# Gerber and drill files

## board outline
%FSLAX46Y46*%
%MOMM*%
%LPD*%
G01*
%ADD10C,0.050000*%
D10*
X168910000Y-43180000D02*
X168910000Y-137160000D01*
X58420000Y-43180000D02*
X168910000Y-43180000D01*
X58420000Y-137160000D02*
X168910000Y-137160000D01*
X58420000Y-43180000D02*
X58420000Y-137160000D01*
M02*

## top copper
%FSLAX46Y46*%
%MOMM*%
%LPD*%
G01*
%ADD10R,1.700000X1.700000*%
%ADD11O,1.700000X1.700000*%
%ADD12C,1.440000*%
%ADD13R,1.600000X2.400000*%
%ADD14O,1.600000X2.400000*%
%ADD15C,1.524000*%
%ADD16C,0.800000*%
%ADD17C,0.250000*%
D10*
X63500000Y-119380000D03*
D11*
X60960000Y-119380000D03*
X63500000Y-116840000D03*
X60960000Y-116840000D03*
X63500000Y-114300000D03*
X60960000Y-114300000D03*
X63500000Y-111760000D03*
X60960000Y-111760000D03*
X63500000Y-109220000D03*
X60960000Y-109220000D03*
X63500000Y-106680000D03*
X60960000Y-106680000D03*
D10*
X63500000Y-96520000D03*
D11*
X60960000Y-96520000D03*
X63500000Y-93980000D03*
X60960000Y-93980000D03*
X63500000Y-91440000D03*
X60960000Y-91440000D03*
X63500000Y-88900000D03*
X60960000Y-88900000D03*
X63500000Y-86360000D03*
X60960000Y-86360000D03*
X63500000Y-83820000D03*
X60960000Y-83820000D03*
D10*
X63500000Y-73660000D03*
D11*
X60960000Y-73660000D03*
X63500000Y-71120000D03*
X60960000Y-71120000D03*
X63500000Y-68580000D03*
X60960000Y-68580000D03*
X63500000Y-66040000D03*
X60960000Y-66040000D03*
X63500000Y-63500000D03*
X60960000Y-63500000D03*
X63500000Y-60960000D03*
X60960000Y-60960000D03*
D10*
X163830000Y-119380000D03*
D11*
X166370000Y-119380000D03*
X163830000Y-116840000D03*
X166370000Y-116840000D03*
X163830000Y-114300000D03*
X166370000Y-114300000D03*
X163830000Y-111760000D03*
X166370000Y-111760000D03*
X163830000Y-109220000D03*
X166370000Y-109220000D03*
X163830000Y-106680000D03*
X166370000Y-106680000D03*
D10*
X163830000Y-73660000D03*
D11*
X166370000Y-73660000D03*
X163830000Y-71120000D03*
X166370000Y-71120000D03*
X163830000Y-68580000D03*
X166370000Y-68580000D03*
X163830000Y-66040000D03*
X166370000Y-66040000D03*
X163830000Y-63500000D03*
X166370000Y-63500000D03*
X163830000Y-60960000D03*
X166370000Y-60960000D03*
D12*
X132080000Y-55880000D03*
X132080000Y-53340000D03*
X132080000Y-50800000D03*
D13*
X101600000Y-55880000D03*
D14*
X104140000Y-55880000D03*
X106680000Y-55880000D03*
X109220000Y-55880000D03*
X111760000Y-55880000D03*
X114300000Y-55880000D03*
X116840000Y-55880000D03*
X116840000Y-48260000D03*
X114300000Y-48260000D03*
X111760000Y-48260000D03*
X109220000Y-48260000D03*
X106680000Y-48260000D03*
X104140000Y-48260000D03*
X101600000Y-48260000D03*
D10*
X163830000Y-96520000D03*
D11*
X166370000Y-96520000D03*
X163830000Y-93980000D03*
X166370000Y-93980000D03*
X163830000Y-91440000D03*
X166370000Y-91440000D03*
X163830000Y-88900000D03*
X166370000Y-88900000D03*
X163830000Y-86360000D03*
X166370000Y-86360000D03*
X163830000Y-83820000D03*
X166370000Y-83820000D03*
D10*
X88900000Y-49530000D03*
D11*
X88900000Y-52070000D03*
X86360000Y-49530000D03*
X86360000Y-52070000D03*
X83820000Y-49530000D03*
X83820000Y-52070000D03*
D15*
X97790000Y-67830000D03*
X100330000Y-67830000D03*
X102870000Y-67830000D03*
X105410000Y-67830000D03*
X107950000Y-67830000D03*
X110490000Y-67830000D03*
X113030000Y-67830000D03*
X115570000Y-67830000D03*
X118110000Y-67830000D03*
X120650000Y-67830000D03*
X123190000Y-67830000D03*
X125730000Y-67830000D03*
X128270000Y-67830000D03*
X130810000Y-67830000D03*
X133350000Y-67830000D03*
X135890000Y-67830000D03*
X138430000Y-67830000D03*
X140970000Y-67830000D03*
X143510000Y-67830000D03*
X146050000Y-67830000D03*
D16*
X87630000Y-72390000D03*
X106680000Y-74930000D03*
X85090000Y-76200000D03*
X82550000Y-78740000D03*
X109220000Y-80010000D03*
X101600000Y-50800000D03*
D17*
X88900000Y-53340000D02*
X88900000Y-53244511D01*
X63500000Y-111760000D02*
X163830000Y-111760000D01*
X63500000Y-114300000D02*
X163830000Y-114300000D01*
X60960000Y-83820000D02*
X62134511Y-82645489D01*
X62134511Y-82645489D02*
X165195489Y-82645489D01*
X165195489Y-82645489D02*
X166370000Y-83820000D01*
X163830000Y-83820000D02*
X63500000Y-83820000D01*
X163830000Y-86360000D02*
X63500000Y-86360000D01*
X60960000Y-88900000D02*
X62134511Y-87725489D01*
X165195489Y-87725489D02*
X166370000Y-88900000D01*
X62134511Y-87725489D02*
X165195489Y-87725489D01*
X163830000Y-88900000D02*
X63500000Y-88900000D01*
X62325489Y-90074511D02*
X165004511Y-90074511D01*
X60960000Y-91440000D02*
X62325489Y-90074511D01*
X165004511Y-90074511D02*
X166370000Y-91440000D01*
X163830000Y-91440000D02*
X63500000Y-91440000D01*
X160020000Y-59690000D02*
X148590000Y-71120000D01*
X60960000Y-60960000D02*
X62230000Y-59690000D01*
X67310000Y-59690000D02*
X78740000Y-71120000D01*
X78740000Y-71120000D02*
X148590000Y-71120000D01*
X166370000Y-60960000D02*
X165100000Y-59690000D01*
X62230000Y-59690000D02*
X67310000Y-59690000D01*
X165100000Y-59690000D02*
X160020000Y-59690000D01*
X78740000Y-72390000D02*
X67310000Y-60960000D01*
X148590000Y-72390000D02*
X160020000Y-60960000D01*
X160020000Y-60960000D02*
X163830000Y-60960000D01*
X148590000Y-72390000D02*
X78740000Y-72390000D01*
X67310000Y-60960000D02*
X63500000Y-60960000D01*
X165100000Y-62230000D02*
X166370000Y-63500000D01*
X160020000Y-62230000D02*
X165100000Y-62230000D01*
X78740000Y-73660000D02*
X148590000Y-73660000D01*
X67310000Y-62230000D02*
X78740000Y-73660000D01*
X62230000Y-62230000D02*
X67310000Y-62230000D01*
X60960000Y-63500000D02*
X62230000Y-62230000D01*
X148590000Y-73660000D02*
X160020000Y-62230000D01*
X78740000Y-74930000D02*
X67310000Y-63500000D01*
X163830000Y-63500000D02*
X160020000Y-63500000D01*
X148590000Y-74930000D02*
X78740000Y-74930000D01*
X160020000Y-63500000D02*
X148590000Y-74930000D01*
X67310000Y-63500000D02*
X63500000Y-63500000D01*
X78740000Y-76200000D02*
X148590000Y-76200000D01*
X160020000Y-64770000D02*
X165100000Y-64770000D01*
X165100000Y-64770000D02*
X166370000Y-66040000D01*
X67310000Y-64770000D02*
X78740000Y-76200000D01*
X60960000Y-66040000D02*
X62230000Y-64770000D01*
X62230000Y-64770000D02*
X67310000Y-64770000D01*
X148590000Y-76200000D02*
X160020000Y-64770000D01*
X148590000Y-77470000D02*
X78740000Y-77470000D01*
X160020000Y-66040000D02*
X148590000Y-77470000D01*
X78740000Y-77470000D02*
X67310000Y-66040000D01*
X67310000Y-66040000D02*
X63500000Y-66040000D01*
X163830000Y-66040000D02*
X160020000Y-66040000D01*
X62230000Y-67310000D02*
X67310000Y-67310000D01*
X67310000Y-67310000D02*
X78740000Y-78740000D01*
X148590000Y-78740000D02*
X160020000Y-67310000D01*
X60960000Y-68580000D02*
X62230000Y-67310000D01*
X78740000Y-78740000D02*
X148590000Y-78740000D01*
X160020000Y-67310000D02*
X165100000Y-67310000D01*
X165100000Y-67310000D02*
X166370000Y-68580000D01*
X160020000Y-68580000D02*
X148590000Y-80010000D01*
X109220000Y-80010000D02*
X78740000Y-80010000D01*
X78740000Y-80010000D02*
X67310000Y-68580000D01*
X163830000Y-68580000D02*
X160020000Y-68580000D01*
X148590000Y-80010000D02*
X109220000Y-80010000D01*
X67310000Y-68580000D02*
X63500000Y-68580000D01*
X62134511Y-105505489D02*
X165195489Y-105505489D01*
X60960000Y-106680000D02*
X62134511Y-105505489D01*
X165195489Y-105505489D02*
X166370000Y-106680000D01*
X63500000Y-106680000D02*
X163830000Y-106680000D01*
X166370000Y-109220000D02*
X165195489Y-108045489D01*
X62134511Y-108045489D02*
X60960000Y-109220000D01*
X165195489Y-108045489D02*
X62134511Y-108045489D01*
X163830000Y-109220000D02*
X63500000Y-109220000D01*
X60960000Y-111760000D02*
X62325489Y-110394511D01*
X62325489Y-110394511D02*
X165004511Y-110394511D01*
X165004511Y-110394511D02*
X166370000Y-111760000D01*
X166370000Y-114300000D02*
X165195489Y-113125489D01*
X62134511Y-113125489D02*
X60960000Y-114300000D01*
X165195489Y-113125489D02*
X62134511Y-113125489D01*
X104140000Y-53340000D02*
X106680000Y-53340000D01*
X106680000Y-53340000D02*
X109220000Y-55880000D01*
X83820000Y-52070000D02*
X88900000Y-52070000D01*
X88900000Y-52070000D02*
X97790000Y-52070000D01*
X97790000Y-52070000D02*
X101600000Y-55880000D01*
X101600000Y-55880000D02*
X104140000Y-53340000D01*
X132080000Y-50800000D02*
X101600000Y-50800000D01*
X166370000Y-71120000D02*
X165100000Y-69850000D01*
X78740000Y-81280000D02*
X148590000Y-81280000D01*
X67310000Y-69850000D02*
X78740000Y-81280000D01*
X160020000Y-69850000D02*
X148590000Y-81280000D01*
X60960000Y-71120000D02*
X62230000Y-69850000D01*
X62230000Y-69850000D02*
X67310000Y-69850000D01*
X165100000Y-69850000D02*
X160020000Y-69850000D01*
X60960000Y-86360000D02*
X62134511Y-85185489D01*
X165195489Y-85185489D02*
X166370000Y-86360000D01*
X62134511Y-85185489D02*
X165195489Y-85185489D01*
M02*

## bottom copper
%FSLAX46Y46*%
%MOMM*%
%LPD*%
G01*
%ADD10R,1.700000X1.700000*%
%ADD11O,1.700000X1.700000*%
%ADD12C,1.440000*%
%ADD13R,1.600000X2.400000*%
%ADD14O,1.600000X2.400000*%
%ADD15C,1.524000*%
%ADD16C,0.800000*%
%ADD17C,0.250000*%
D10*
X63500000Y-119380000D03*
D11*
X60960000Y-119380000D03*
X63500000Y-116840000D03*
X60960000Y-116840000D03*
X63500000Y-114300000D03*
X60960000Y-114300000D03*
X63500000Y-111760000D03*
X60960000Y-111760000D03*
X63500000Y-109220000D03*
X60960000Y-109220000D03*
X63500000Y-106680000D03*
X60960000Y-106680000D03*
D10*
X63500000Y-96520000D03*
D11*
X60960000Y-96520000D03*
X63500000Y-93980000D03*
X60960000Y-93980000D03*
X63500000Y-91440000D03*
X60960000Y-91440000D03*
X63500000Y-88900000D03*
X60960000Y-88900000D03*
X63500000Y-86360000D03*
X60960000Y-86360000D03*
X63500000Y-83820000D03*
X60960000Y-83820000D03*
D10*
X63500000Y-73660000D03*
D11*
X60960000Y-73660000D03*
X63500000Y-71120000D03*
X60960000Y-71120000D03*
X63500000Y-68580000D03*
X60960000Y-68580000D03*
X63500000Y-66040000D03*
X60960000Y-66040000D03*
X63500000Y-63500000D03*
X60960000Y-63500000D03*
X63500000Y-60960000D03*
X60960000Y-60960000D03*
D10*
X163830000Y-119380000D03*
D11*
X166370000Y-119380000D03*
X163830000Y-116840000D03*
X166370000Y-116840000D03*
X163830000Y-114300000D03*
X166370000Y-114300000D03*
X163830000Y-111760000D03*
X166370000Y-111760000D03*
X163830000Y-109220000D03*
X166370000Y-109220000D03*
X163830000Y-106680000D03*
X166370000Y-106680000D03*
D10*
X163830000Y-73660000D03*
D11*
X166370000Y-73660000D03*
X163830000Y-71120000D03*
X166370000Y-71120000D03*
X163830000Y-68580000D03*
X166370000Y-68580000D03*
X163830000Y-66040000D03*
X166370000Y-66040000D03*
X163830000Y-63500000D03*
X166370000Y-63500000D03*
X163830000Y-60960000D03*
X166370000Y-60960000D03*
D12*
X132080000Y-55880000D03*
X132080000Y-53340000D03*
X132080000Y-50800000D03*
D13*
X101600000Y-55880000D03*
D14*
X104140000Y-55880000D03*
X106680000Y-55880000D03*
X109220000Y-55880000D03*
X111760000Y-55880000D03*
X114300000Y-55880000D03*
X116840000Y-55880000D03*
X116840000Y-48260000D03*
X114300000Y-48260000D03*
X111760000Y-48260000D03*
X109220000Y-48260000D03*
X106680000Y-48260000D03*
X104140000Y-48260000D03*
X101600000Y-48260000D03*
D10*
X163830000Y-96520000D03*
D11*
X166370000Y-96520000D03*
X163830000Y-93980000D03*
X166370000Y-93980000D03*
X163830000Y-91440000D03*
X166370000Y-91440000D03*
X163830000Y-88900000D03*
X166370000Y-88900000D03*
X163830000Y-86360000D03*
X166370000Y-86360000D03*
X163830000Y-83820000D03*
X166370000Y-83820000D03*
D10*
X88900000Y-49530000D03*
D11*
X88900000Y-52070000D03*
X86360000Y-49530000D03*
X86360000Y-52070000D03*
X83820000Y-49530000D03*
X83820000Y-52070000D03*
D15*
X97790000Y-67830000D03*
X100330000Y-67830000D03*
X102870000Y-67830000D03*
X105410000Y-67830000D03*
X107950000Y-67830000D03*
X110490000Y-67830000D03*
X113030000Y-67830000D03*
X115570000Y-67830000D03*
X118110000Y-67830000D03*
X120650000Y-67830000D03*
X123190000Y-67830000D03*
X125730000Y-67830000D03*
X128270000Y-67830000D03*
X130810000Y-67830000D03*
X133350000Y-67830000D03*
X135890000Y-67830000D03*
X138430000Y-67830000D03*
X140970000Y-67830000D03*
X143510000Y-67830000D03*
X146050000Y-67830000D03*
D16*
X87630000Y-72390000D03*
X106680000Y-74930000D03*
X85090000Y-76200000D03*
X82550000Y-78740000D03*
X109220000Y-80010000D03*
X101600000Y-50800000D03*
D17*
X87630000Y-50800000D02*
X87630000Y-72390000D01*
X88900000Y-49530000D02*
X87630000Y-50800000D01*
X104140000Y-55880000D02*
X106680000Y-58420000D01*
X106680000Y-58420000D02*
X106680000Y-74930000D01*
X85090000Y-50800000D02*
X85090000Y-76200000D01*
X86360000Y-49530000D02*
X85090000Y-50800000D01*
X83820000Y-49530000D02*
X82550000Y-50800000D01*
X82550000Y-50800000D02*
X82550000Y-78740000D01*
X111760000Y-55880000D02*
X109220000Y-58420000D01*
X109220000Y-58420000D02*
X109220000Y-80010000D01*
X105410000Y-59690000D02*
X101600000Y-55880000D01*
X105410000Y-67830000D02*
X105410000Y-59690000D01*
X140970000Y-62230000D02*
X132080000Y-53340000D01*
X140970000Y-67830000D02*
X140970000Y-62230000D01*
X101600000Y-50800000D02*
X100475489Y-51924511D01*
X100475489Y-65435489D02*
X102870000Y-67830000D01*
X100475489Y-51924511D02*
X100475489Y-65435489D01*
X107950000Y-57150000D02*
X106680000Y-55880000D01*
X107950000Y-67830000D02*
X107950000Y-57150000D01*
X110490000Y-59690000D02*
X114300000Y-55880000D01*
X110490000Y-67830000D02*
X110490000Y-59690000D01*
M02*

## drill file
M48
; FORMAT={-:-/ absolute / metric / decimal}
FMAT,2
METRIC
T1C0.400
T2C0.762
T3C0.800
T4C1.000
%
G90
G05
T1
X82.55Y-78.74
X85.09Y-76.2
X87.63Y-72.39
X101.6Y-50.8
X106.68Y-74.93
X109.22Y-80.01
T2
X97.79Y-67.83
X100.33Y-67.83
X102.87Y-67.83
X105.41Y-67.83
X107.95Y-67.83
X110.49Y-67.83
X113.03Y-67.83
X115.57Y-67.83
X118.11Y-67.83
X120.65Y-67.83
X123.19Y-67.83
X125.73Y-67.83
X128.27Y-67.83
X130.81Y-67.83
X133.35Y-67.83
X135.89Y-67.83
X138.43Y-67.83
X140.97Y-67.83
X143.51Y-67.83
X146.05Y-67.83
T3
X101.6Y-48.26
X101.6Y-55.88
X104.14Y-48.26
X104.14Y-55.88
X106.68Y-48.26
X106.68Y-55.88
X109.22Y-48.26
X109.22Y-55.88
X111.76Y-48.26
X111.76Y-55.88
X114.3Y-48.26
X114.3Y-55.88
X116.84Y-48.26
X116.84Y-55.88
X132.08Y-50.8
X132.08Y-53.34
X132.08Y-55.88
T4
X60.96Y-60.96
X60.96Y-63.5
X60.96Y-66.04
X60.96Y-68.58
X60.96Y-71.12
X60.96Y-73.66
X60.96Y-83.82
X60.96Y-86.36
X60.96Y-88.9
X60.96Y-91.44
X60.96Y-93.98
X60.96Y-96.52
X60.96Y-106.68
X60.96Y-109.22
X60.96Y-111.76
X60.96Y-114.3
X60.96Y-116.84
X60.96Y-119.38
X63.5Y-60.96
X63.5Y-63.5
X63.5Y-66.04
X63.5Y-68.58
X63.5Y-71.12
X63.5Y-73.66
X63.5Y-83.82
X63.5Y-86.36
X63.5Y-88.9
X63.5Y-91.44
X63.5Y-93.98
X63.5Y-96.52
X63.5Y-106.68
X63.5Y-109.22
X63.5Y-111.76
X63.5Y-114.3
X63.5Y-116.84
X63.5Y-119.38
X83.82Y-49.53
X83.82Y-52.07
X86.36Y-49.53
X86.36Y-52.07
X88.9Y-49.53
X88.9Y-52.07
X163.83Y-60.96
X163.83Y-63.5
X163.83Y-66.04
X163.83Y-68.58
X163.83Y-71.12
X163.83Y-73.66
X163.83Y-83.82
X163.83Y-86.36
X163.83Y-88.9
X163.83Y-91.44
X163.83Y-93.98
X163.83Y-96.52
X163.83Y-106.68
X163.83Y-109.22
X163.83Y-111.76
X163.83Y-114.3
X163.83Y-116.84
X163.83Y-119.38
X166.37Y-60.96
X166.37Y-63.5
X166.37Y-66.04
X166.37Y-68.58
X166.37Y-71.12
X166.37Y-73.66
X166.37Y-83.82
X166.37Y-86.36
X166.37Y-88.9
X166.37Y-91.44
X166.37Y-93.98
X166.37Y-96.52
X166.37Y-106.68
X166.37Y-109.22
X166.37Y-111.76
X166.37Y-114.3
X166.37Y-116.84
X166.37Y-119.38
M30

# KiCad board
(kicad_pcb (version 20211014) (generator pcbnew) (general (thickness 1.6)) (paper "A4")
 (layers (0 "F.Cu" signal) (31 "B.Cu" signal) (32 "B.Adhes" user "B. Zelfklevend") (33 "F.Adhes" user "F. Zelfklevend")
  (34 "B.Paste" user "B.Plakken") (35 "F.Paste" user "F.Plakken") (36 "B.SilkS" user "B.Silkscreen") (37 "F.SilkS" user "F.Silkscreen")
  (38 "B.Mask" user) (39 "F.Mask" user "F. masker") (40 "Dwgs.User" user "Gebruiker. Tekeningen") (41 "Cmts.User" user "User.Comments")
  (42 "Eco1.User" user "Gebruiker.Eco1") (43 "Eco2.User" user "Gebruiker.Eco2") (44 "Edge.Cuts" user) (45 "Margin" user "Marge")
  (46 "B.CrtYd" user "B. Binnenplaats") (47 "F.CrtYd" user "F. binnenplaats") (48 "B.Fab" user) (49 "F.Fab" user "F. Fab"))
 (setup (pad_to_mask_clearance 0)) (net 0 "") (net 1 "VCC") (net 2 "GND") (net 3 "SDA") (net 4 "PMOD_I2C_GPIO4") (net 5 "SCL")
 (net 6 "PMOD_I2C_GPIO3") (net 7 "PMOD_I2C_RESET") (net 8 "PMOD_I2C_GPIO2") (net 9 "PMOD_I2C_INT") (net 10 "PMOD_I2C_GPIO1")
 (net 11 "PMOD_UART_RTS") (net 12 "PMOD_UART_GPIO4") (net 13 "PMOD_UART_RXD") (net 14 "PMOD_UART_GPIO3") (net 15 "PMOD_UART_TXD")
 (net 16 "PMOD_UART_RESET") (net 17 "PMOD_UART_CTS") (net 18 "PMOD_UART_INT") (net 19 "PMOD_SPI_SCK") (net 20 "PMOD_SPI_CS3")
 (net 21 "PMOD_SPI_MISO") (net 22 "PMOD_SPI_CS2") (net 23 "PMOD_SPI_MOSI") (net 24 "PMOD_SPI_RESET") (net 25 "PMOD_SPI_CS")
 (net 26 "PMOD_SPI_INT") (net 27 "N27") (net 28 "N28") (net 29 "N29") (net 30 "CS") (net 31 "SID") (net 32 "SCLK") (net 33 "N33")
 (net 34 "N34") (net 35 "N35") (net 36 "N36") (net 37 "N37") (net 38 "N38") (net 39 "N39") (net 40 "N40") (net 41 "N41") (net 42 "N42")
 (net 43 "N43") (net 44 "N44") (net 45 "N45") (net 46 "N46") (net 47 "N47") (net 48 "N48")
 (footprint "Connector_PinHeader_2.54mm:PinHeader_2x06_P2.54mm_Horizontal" (layer "F.Cu") (at 63.5 119.38 180)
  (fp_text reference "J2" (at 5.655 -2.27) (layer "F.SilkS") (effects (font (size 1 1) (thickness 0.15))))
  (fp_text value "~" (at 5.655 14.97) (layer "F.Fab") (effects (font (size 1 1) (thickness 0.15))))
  (pad "1" thru_hole rect (at 0 0 180) (size 1.7 1.7) (drill 1) (layers *.Cu *.Mask) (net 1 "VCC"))
  (pad "2" thru_hole oval (at 2.54 0 180) (size 1.7 1.7) (drill 1) (layers *.Cu *.Mask) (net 1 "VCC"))
  (pad "3" thru_hole oval (at 0 2.54 180) (size 1.7 1.7) (drill 1) (layers *.Cu *.Mask) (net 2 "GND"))
  (pad "4" thru_hole oval (at 2.54 2.54 180) (size 1.7 1.7) (drill 1) (layers *.Cu *.Mask) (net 2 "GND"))
  (pad "5" thru_hole oval (at 0 5.08 180) (size 1.7 1.7) (drill 1) (layers *.Cu *.Mask) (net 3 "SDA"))
  (pad "6" thru_hole oval (at 2.54 5.08 180) (size 1.7 1.7) (drill 1) (layers *.Cu *.Mask) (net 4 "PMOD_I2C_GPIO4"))
  (pad "7" thru_hole oval (at 0 7.62 180) (size 1.7 1.7) (drill 1) (layers *.Cu *.Mask) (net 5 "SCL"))
  (pad "8" thru_hole oval (at 2.54 7.62 180) (size 1.7 1.7) (drill 1) (layers *.Cu *.Mask) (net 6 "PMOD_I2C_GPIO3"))
  (pad "9" thru_hole oval (at 0 10.16 180) (size 1.7 1.7) (drill 1) (layers *.Cu *.Mask) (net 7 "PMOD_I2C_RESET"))
  (pad "10" thru_hole oval (at 2.54 10.16 180) (size 1.7 1.7) (drill 1) (layers *.Cu *.Mask) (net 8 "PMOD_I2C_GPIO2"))
  (pad "11" thru_hole oval (at 0 12.7 180) (size 1.7 1.7) (drill 1) (layers *.Cu *.Mask) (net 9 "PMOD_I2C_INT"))
  (pad "12" thru_hole oval (at 2.54 12.7 180) (size 1.7 1.7) (drill 1) (layers *.Cu *.Mask) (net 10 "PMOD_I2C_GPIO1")))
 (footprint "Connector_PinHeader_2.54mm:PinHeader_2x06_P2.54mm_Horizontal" (layer "F.Cu") (at 63.5 96.52 180)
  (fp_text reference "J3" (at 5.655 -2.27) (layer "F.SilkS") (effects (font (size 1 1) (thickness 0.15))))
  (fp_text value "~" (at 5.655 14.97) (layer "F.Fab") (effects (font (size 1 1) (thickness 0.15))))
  (pad "1" thru_hole rect (at 0 0 180) (size 1.7 1.7) (drill 1) (layers *.Cu *.Mask) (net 1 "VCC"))
  (pad "2" thru_hole oval (at 2.54 0 180) (size 1.7 1.7) (drill 1) (layers *.Cu *.Mask) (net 1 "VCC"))
  (pad "3" thru_hole oval (at 0 2.54 180) (size 1.7 1.7) (drill 1) (layers *.Cu *.Mask) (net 2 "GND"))
  (pad "4" thru_hole oval (at 2.54 2.54 180) (size 1.7 1.7) (drill 1) (layers *.Cu *.Mask) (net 2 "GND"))
  (pad "5" thru_hole oval (at 0 5.08 180) (size 1.7 1.7) (drill 1) (layers *.Cu *.Mask) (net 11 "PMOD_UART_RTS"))
  (pad "6" thru_hole oval (at 2.54 5.08 180) (size 1.7 1.7) (drill 1) (layers *.Cu *.Mask) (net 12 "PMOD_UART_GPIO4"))
  (pad "7" thru_hole oval (at 0 7.62 180) (size 1.7 1.7) (drill 1) (layers *.Cu *.Mask) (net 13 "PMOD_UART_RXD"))
  (pad "8" thru_hole oval (at 2.54 7.62 180) (size 1.7 1.7) (drill 1) (layers *.Cu *.Mask) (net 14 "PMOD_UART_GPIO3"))
  (pad "9" thru_hole oval (at 0 10.16 180) (size 1.7 1.7) (drill 1) (layers *.Cu *.Mask) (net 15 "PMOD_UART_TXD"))
  (pad "10" thru_hole oval (at 2.54 10.16 180) (size 1.7 1.7) (drill 1) (layers *.Cu *.Mask) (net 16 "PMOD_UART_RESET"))
  (pad "11" thru_hole oval (at 0 12.7 180) (size 1.7 1.7) (drill 1) (layers *.Cu *.Mask) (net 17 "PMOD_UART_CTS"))
  (pad "12" thru_hole oval (at 2.54 12.7 180) (size 1.7 1.7) (drill 1) (layers *.Cu *.Mask) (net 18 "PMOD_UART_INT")))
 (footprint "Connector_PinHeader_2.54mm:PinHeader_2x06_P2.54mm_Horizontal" (layer "F.Cu") (at 63.5 73.66 180)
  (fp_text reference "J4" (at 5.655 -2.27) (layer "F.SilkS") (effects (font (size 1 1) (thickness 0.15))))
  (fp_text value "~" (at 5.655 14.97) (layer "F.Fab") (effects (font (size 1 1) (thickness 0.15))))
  (pad "1" thru_hole rect (at 0 0 180) (size 1.7 1.7) (drill 1) (layers *.Cu *.Mask) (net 1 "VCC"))
  (pad "2" thru_hole oval (at 2.54 0 180) (size 1.7 1.7) (drill 1) (layers *.Cu *.Mask) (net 1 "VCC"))
  (pad "3" thru_hole oval (at 0 2.54 180) (size 1.7 1.7) (drill 1) (layers *.Cu *.Mask) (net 2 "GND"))
  (pad "4" thru_hole oval (at 2.54 2.54 180) (size 1.7 1.7) (drill 1) (layers *.Cu *.Mask) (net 2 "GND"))
  (pad "5" thru_hole oval (at 0 5.08 180) (size 1.7 1.7) (drill 1) (layers *.Cu *.Mask) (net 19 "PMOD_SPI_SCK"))
  (pad "6" thru_hole oval (at 2.54 5.08 180) (size 1.7 1.7) (drill 1) (layers *.Cu *.Mask) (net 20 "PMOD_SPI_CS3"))
  (pad "7" thru_hole oval (at 0 7.62 180) (size 1.7 1.7) (drill 1) (layers *.Cu *.Mask) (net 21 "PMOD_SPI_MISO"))
  (pad "8" thru_hole oval (at 2.54 7.62 180) (size 1.7 1.7) (drill 1) (layers *.Cu *.Mask) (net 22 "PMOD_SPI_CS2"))
  (pad "9" thru_hole oval (at 0 10.16 180) (size 1.7 1.7) (drill 1) (layers *.Cu *.Mask) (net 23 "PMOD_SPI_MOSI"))
  (pad "10" thru_hole oval (at 2.54 10.16 180) (size 1.7 1.7) (drill 1) (layers *.Cu *.Mask) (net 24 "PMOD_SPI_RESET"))
  (pad "11" thru_hole oval (at 0 12.7 180) (size 1.7 1.7) (drill 1) (layers *.Cu *.Mask) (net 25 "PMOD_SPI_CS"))
  (pad "12" thru_hole oval (at 2.54 12.7 180) (size 1.7 1.7) (drill 1) (layers *.Cu *.Mask) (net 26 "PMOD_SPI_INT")))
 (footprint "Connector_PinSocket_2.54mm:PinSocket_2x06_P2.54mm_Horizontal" (layer "F.Cu") (at 163.83 119.38 180)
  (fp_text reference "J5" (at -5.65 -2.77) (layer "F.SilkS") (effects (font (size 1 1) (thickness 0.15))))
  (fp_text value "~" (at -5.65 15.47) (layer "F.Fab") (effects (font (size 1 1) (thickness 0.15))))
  (pad "1" thru_hole rect (at 0 0 180) (size 1.7 1.7) (drill 1) (layers *.Cu *.Mask) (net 1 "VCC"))
  (pad "2" thru_hole oval (at -2.54 0 180) (size 1.7 1.7) (drill 1) (layers *.Cu *.Mask) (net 1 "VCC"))
  (pad "3" thru_hole oval (at 0 2.54 180) (size 1.7 1.7) (drill 1) (layers *.Cu *.Mask) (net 2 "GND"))
  (pad "4" thru_hole oval (at -2.54 2.54 180) (size 1.7 1.7) (drill 1) (layers *.Cu *.Mask) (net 2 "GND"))
  (pad "5" thru_hole oval (at 0 5.08 180) (size 1.7 1.7) (drill 1) (layers *.Cu *.Mask) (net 3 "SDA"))
  (pad "6" thru_hole oval (at -2.54 5.08 180) (size 1.7 1.7) (drill 1) (layers *.Cu *.Mask) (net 4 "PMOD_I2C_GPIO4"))
  (pad "7" thru_hole oval (at 0 7.62 180) (size 1.7 1.7) (drill 1) (layers *.Cu *.Mask) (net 5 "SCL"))
  (pad "8" thru_hole oval (at -2.54 7.62 180) (size 1.7 1.7) (drill 1) (layers *.Cu *.Mask) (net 6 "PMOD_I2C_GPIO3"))
  (pad "9" thru_hole oval (at 0 10.16 180) (size 1.7 1.7) (drill 1) (layers *.Cu *.Mask) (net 7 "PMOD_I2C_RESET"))
  (pad "10" thru_hole oval (at -2.54 10.16 180) (size 1.7 1.7) (drill 1) (layers *.Cu *.Mask) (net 8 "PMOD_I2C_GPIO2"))
  (pad "11" thru_hole oval (at 0 12.7 180) (size 1.7 1.7) (drill 1) (layers *.Cu *.Mask) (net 9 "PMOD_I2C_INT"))
  (pad "12" thru_hole oval (at -2.54 12.7 180) (size 1.7 1.7) (drill 1) (layers *.Cu *.Mask) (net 10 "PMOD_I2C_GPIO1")))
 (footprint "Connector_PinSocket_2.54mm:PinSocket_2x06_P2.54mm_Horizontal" (layer "F.Cu") (at 163.83 73.66 180)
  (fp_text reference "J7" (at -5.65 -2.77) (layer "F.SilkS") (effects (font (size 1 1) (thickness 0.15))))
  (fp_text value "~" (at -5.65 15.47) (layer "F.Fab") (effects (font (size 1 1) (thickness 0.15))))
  (pad "1" thru_hole rect (at 0 0 180) (size 1.7 1.7) (drill 1) (layers *.Cu *.Mask) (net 1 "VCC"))
  (pad "2" thru_hole oval (at -2.54 0 180) (size 1.7 1.7) (drill 1) (layers *.Cu *.Mask) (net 1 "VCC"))
  (pad "3" thru_hole oval (at 0 2.54 180) (size 1.7 1.7) (drill 1) (layers *.Cu *.Mask) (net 2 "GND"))
  (pad "4" thru_hole oval (at -2.54 2.54 180) (size 1.7 1.7) (drill 1) (layers *.Cu *.Mask) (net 2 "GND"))
  (pad "5" thru_hole oval (at 0 5.08 180) (size 1.7 1.7) (drill 1) (layers *.Cu *.Mask) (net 19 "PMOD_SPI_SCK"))
  (pad "6" thru_hole oval (at -2.54 5.08 180) (size 1.7 1.7) (drill 1) (layers *.Cu *.Mask) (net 20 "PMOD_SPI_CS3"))
  (pad "7" thru_hole oval (at 0 7.62 180) (size 1.7 1.7) (drill 1) (layers *.Cu *.Mask) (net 21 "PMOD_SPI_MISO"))
  (pad "8" thru_hole oval (at -2.54 7.62 180) (size 1.7 1.7) (drill 1) (layers *.Cu *.Mask) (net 22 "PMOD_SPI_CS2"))
  (pad "9" thru_hole oval (at 0 10.16 180) (size 1.7 1.7) (drill 1) (layers *.Cu *.Mask) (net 23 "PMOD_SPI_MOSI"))
  (pad "10" thru_hole oval (at -2.54 10.16 180) (size 1.7 1.7) (drill 1) (layers *.Cu *.Mask) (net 24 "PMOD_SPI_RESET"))
  (pad "11" thru_hole oval (at 0 12.7 180) (size 1.7 1.7) (drill 1) (layers *.Cu *.Mask) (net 25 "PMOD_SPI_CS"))
  (pad "12" thru_hole oval (at -2.54 12.7 180) (size 1.7 1.7) (drill 1) (layers *.Cu *.Mask) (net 26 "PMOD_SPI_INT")))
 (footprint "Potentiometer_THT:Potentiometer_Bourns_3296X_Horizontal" (layer "F.Cu") (at 132.08 55.88 -90)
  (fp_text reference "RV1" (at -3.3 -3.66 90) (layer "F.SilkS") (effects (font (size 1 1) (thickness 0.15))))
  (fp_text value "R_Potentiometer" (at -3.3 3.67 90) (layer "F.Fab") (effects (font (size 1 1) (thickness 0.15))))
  (pad "1" thru_hole circle (at 0 0 270) (size 1.44 1.44) (drill 0.8) (layers *.Cu *.Mask) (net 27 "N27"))
  (pad "2" thru_hole circle (at -2.54 0 270) (size 1.44 1.44) (drill 0.8) (layers *.Cu *.Mask) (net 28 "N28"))
  (pad "3" thru_hole circle (at -5.08 0 270) (size 1.44 1.44) (drill 0.8) (layers *.Cu *.Mask) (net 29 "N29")))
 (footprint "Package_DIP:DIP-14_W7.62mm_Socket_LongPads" (layer "F.Cu") (at 101.6 55.88 90)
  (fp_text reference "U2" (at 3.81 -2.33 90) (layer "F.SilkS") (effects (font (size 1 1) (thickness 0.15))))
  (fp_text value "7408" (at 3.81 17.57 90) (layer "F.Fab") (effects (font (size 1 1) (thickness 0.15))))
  (pad "1" thru_hole rect (at 0 0 90) (size 2.4 1.6) (drill 0.8) (layers *.Cu *.Mask) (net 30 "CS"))
  (pad "2" thru_hole oval (at 0 2.54 90) (size 2.4 1.6) (drill 0.8) (layers *.Cu *.Mask) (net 23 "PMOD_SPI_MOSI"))
  (pad "3" thru_hole oval (at 0 5.08 90) (size 2.4 1.6) (drill 0.8) (layers *.Cu *.Mask) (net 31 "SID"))
  (pad "4" thru_hole oval (at 0 7.62 90) (size 2.4 1.6) (drill 0.8) (layers *.Cu *.Mask) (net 30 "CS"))
  (pad "5" thru_hole oval (at 0 10.16 90) (size 2.4 1.6) (drill 0.8) (layers *.Cu *.Mask) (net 19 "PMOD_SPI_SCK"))
  (pad "6" thru_hole oval (at 0 12.7 90) (size 2.4 1.6) (drill 0.8) (layers *.Cu *.Mask) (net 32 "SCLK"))
  (pad "7" thru_hole oval (at 0 15.24 90) (size 2.4 1.6) (drill 0.8) (layers *.Cu *.Mask) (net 2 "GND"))
  (pad "8" thru_hole oval (at 7.62 15.24 90) (size 2.4 1.6) (drill 0.8) (layers *.Cu *.Mask) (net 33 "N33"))
  (pad "9" thru_hole oval (at 7.62 12.7 90) (size 2.4 1.6) (drill 0.8) (layers *.Cu *.Mask) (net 2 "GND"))
  (pad "10" thru_hole oval (at 7.62 10.16 90) (size 2.4 1.6) (drill 0.8) (layers *.Cu *.Mask) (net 2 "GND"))
  (pad "11" thru_hole oval (at 7.62 7.62 90) (size 2.4 1.6) (drill 0.8) (layers *.Cu *.Mask) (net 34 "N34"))
  (pad "12" thru_hole oval (at 7.62 5.08 90) (size 2.4 1.6) (drill 0.8) (layers *.Cu *.Mask) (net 2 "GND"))
  (pad "13" thru_hole oval (at 7.62 2.54 90) (size 2.4 1.6) (drill 0.8) (layers *.Cu *.Mask) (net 2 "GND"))
  (pad "14" thru_hole oval (at 7.62 0 90) (size 2.4 1.6) (drill 0.8) (layers *.Cu *.Mask) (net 1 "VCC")))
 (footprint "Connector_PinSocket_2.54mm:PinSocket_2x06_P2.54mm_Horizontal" (layer "F.Cu") (at 163.83 96.52 180)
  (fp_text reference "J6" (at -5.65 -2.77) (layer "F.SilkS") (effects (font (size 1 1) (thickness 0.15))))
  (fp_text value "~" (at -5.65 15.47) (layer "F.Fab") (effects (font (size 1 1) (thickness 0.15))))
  (pad "1" thru_hole rect (at 0 0 180) (size 1.7 1.7) (drill 1) (layers *.Cu *.Mask) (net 1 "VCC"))
  (pad "2" thru_hole oval (at -2.54 0 180) (size 1.7 1.7) (drill 1) (layers *.Cu *.Mask) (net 1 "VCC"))
  (pad "3" thru_hole oval (at 0 2.54 180) (size 1.7 1.7) (drill 1) (layers *.Cu *.Mask) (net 2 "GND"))
  (pad "4" thru_hole oval (at -2.54 2.54 180) (size 1.7 1.7) (drill 1) (layers *.Cu *.Mask) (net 2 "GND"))
  (pad "5" thru_hole oval (at 0 5.08 180) (size 1.7 1.7) (drill 1) (layers *.Cu *.Mask) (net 11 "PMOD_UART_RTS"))
  (pad "6" thru_hole oval (at -2.54 5.08 180) (size 1.7 1.7) (drill 1) (layers *.Cu *.Mask) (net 12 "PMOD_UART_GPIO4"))
  (pad "7" thru_hole oval (at 0 7.62 180) (size 1.7 1.7) (drill 1) (layers *.Cu *.Mask) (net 13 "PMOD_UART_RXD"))
  (pad "8" thru_hole oval (at -2.54 7.62 180) (size 1.7 1.7) (drill 1) (layers *.Cu *.Mask) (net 14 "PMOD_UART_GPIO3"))
  (pad "9" thru_hole oval (at 0 10.16 180) (size 1.7 1.7) (drill 1) (layers *.Cu *.Mask) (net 15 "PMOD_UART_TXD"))
  (pad "10" thru_hole oval (at -2.54 10.16 180) (size 1.7 1.7) (drill 1) (layers *.Cu *.Mask) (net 16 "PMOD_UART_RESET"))
  (pad "11" thru_hole oval (at 0 12.7 180) (size 1.7 1.7) (drill 1) (layers *.Cu *.Mask) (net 17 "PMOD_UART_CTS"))
  (pad "12" thru_hole oval (at -2.54 12.7 180) (size 1.7 1.7) (drill 1) (layers *.Cu *.Mask) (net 18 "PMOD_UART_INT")))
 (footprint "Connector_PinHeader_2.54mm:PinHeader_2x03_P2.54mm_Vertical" (layer "F.Cu") (at 88.9 49.53 -90)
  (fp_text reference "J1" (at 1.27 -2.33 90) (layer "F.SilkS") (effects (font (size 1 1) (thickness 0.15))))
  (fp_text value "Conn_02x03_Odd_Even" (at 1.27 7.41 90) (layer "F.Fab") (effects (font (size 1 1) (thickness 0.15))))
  (pad "1" thru_hole rect (at 0 0 270) (size 1.7 1.7) (drill 1) (layers *.Cu *.Mask) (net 25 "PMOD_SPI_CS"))
  (pad "2" thru_hole oval (at 2.54 0 270) (size 1.7 1.7) (drill 1) (layers *.Cu *.Mask) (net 30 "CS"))
  (pad "3" thru_hole oval (at 0 2.54 270) (size 1.7 1.7) (drill 1) (layers *.Cu *.Mask) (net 22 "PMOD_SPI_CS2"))
  (pad "4" thru_hole oval (at 2.54 2.54 270) (size 1.7 1.7) (drill 1) (layers *.Cu *.Mask) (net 30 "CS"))
  (pad "5" thru_hole oval (at 0 5.08 270) (size 1.7 1.7) (drill 1) (layers *.Cu *.Mask) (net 20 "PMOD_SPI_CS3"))
  (pad "6" thru_hole oval (at 2.54 5.08 270) (size 1.7 1.7) (drill 1) (layers *.Cu *.Mask) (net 30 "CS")))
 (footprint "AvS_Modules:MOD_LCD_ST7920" (layer "F.Cu") (at 113.59 100.33 180)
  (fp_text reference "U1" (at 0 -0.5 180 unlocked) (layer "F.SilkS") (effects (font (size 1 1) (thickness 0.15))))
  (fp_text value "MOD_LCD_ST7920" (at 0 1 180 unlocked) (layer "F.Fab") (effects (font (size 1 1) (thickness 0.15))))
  (pad "1" thru_hole circle (at 15.8 32.5 180) (size 1.524 1.524) (drill 0.762) (layers *.Cu *.Mask) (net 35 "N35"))
  (pad "2" thru_hole circle (at 13.26 32.5 180) (size 1.524 1.524) (drill 0.762) (layers *.Cu *.Mask) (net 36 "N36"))
  (pad "3" thru_hole circle (at 10.72 32.5 180) (size 1.524 1.524) (drill 0.762) (layers *.Cu *.Mask) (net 29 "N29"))
  (pad "4" thru_hole circle (at 8.18 32.5 180) (size 1.524 1.524) (drill 0.762) (layers *.Cu *.Mask) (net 30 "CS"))
  (pad "5" thru_hole circle (at 5.64 32.5 180) (size 1.524 1.524) (drill 0.762) (layers *.Cu *.Mask) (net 31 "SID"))
  (pad "6" thru_hole circle (at 3.1 32.5 180) (size 1.524 1.524) (drill 0.762) (layers *.Cu *.Mask) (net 32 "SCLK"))
  (pad "7" thru_hole circle (at 0.56 32.5 180) (size 1.524 1.524) (drill 0.762) (layers *.Cu *.Mask) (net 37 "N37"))
  (pad "8" thru_hole circle (at -1.98 32.5 180) (size 1.524 1.524) (drill 0.762) (layers *.Cu *.Mask) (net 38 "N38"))
  (pad "9" thru_hole circle (at -4.52 32.5 180) (size 1.524 1.524) (drill 0.762) (layers *.Cu *.Mask) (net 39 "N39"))
  (pad "10" thru_hole circle (at -7.06 32.5 180) (size 1.524 1.524) (drill 0.762) (layers *.Cu *.Mask) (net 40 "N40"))
  (pad "11" thru_hole circle (at -9.6 32.5 180) (size 1.524 1.524) (drill 0.762) (layers *.Cu *.Mask) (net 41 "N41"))
  (pad "12" thru_hole circle (at -12.14 32.5 180) (size 1.524 1.524) (drill 0.762) (layers *.Cu *.Mask) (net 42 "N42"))
  (pad "13" thru_hole circle (at -14.68 32.5 180) (size 1.524 1.524) (drill 0.762) (layers *.Cu *.Mask) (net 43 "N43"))
  (pad "14" thru_hole circle (at -17.22 32.5 180) (size 1.524 1.524) (drill 0.762) (layers *.Cu *.Mask) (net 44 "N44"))
  (pad "15" thru_hole circle (at -19.76 32.5 180) (size 1.524 1.524) (drill 0.762) (layers *.Cu *.Mask) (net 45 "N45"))
  (pad "16" thru_hole circle (at -22.3 32.5 180) (size 1.524 1.524) (drill 0.762) (layers *.Cu *.Mask))
  (pad "17" thru_hole circle (at -24.84 32.5 180) (size 1.524 1.524) (drill 0.762) (layers *.Cu *.Mask) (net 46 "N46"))
  (pad "18" thru_hole circle (at -27.38 32.5 180) (size 1.524 1.524) (drill 0.762) (layers *.Cu *.Mask) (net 28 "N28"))
  (pad "19" thru_hole circle (at -29.92 32.5 180) (size 1.524 1.524) (drill 0.762) (layers *.Cu *.Mask) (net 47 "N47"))
  (pad "20" thru_hole circle (at -32.46 32.5 180) (size 1.524 1.524) (drill 0.762) (layers *.Cu *.Mask) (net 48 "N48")))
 (gr_line (start 168.91 43.18) (end 168.91 137.16) (layer "Edge.Cuts") (width 0.05))
 (gr_line (start 58.42 43.18) (end 168.91 43.18) (layer "Edge.Cuts") (width 0.05))
 (gr_line (start 58.42 137.16) (end 168.91 137.16) (layer "Edge.Cuts") (width 0.05))
 (gr_line (start 58.42 43.18) (end 58.42 137.16) (layer "Edge.Cuts") (width 0.05))
 (segment (start 88.9 53.34) (end 88.9 53.244511) (width 0.25) (layer "F.Cu") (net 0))
 (segment (start 63.5 111.76) (end 163.83 111.76) (width 0.25) (layer "F.Cu") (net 5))
 (segment (start 63.5 114.3) (end 163.83 114.3) (width 0.25) (layer "F.Cu") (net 3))
 (segment (start 60.96 83.82) (end 62.134511 82.645489) (width 0.25) (layer "F.Cu") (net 18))
 (segment (start 62.134511 82.645489) (end 165.195489 82.645489) (width 0.25) (layer "F.Cu") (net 18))
 (segment (start 165.195489 82.645489) (end 166.37 83.82) (width 0.25) (layer "F.Cu") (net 18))
 (segment (start 163.83 83.82) (end 63.5 83.82) (width 0.25) (layer "F.Cu") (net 17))
 (segment (start 163.83 86.36) (end 63.5 86.36) (width 0.25) (layer "F.Cu") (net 15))
 (segment (start 60.96 88.9) (end 62.134511 87.725489) (width 0.25) (layer "F.Cu") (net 14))
 (segment (start 165.195489 87.725489) (end 166.37 88.9) (width 0.25) (layer "F.Cu") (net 14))
 (segment (start 62.134511 87.725489) (end 165.195489 87.725489) (width 0.25) (layer "F.Cu") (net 14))
 (segment (start 163.83 88.9) (end 63.5 88.9) (width 0.25) (layer "F.Cu") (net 13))
 (segment (start 62.325489 90.074511) (end 165.004511 90.074511) (width 0.25) (layer "F.Cu") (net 12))
 (segment (start 60.96 91.44) (end 62.325489 90.074511) (width 0.25) (layer "F.Cu") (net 12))
 (segment (start 165.004511 90.074511) (end 166.37 91.44) (width 0.25) (layer "F.Cu") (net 12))
 (segment (start 163.83 91.44) (end 63.5 91.44) (width 0.25) (layer "F.Cu") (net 11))
 (segment (start 160.02 59.69) (end 148.59 71.12) (width 0.25) (layer "F.Cu") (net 26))
 (segment (start 60.96 60.96) (end 62.23 59.69) (width 0.25) (layer "F.Cu") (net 26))
 (segment (start 67.31 59.69) (end 78.74 71.12) (width 0.25) (layer "F.Cu") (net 26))
 (segment (start 78.74 71.12) (end 148.59 71.12) (width 0.25) (layer "F.Cu") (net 26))
 (segment (start 166.37 60.96) (end 165.1 59.69) (width 0.25) (layer "F.Cu") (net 26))
 (segment (start 62.23 59.69) (end 67.31 59.69) (width 0.25) (layer "F.Cu") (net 26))
 (segment (start 165.1 59.69) (end 160.02 59.69) (width 0.25) (layer "F.Cu") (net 26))
 (segment (start 78.74 72.39) (end 67.31 60.96) (width 0.25) (layer "F.Cu") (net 25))
 (segment (start 148.59 72.39) (end 160.02 60.96) (width 0.25) (layer "F.Cu") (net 25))
 (segment (start 160.02 60.96) (end 163.83 60.96) (width 0.25) (layer "F.Cu") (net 25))
 (segment (start 148.59 72.39) (end 78.74 72.39) (width 0.25) (layer "F.Cu") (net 25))
 (segment (start 67.31 60.96) (end 63.5 60.96) (width 0.25) (layer "F.Cu") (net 25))
 (via (at 87.63 72.39) (size 0.8) (drill 0.4) (layers "F.Cu" "B.Cu") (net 25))
 (segment (start 87.63 50.8) (end 87.63 72.39) (width 0.25) (layer "B.Cu") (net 25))
 (segment (start 88.9 49.53) (end 87.63 50.8) (width 0.25) (layer "B.Cu") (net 25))
 (segment (start 165.1 62.23) (end 166.37 63.5) (width 0.25) (layer "F.Cu") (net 24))
 (segment (start 160.02 62.23) (end 165.1 62.23) (width 0.25) (layer "F.Cu") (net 24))
 (segment (start 78.74 73.66) (end 148.59 73.66) (width 0.25) (layer "F.Cu") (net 24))
 (segment (start 67.31 62.23) (end 78.74 73.66) (width 0.25) (layer "F.Cu") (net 24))
 (segment (start 62.23 62.23) (end 67.31 62.23) (width 0.25) (layer "F.Cu") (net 24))
 (segment (start 60.96 63.5) (end 62.23 62.23) (width 0.25) (layer "F.Cu") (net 24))
 (segment (start 148.59 73.66) (end 160.02 62.23) (width 0.25) (layer "F.Cu") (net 24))
 (segment (start 78.74 74.93) (end 67.31 63.5) (width 0.25) (layer "F.Cu") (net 23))
 (segment (start 163.83 63.5) (end 160.02 63.5) (width 0.25) (layer "F.Cu") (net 23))
 (segment (start 148.59 74.93) (end 78.74 74.93) (width 0.25) (layer "F.Cu") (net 23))
 (segment (start 160.02 63.5) (end 148.59 74.93) (width 0.25) (layer "F.Cu") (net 23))
 (segment (start 67.31 63.5) (end 63.5 63.5) (width 0.25) (layer "F.Cu") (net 23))
 (via (at 106.68 74.93) (size 0.8) (drill 0.4) (layers "F.Cu" "B.Cu") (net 23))
 (segment (start 104.14 55.88) (end 106.68 58.42) (width 0.25) (layer "B.Cu") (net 23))
 (segment (start 106.68 58.42) (end 106.68 74.93) (width 0.25) (layer "B.Cu") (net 23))
 (segment (start 78.74 76.2) (end 148.59 76.2) (width 0.25) (layer "F.Cu") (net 22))
 (segment (start 160.02 64.77) (end 165.1 64.77) (width 0.25) (layer "F.Cu") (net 22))
 (segment (start 165.1 64.77) (end 166.37 66.04) (width 0.25) (layer "F.Cu") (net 22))
 (segment (start 67.31 64.77) (end 78.74 76.2) (width 0.25) (layer "F.Cu") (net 22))
 (segment (start 60.96 66.04) (end 62.23 64.77) (width 0.25) (layer "F.Cu") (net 22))
 (segment (start 62.23 64.77) (end 67.31 64.77) (width 0.25) (layer "F.Cu") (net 22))
 (segment (start 148.59 76.2) (end 160.02 64.77) (width 0.25) (layer "F.Cu") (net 22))
 (via (at 85.09 76.2) (size 0.8) (drill 0.4) (layers "F.Cu" "B.Cu") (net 22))
 (segment (start 85.09 50.8) (end 85.09 76.2) (width 0.25) (layer "B.Cu") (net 22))
 (segment (start 86.36 49.53) (end 85.09 50.8) (width 0.25) (layer "B.Cu") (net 22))
 (segment (start 148.59 77.47) (end 78.74 77.47) (width 0.25) (layer "F.Cu") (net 21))
 (segment (start 160.02 66.04) (end 148.59 77.47) (width 0.25) (layer "F.Cu") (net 21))
 (segment (start 78.74 77.47) (end 67.31 66.04) (width 0.25) (layer "F.Cu") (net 21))
 (segment (start 67.31 66.04) (end 63.5 66.04) (width 0.25) (layer "F.Cu") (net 21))
 (segment (start 163.83 66.04) (end 160.02 66.04) (width 0.25) (layer "F.Cu") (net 21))
 (segment (start 62.23 67.31) (end 67.31 67.31) (width 0.25) (layer "F.Cu") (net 20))
 (segment (start 67.31 67.31) (end 78.74 78.74) (width 0.25) (layer "F.Cu") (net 20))
 (segment (start 148.59 78.74) (end 160.02 67.31) (width 0.25) (layer "F.Cu") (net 20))
 (segment (start 60.96 68.58) (end 62.23 67.31) (width 0.25) (layer "F.Cu") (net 20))
 (segment (start 78.74 78.74) (end 148.59 78.74) (width 0.25) (layer "F.Cu") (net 20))
 (segment (start 160.02 67.31) (end 165.1 67.31) (width 0.25) (layer "F.Cu") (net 20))
 (segment (start 165.1 67.31) (end 166.37 68.58) (width 0.25) (layer "F.Cu") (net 20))
 (via (at 82.55 78.74) (size 0.8) (drill 0.4) (layers "F.Cu" "B.Cu") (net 20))
 (segment (start 83.82 49.53) (end 82.55 50.8) (width 0.25) (layer "B.Cu") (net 20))
 (segment (start 82.55 50.8) (end 82.55 78.74) (width 0.25) (layer "B.Cu") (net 20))
 (segment (start 160.02 68.58) (end 148.59 80.01) (width 0.25) (layer "F.Cu") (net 19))
 (segment (start 109.22 80.01) (end 78.74 80.01) (width 0.25) (layer "F.Cu") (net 19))
 (segment (start 78.74 80.01) (end 67.31 68.58) (width 0.25) (layer "F.Cu") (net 19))
 (segment (start 163.83 68.58) (end 160.02 68.58) (width 0.25) (layer "F.Cu") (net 19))
 (segment (start 148.59 80.01) (end 109.22 80.01) (width 0.25) (layer "F.Cu") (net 19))
 (segment (start 67.31 68.58) (end 63.5 68.58) (width 0.25) (layer "F.Cu") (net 19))
 (via (at 109.22 80.01) (size 0.8) (drill 0.4) (layers "F.Cu" "B.Cu") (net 19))
 (segment (start 111.76 55.88) (end 109.22 58.42) (width 0.25) (layer "B.Cu") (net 19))
 (segment (start 109.22 58.42) (end 109.22 80.01) (width 0.25) (layer "B.Cu") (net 19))
 (segment (start 62.134511 105.505489) (end 165.195489 105.505489) (width 0.25) (layer "F.Cu") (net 10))
 (segment (start 60.96 106.68) (end 62.134511 105.505489) (width 0.25) (layer "F.Cu") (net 10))
 (segment (start 165.195489 105.505489) (end 166.37 106.68) (width 0.25) (layer "F.Cu") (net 10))
 (segment (start 63.5 106.68) (end 163.83 106.68) (width 0.25) (layer "F.Cu") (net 9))
 (segment (start 166.37 109.22) (end 165.195489 108.045489) (width 0.25) (layer "F.Cu") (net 8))
 (segment (start 62.134511 108.045489) (end 60.96 109.22) (width 0.25) (layer "F.Cu") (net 8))
 (segment (start 165.195489 108.045489) (end 62.134511 108.045489) (width 0.25) (layer "F.Cu") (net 8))
 (segment (start 163.83 109.22) (end 63.5 109.22) (width 0.25) (layer "F.Cu") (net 7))
 (segment (start 60.96 111.76) (end 62.325489 110.394511) (width 0.25) (layer "F.Cu") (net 6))
 (segment (start 62.325489 110.394511) (end 165.004511 110.394511) (width 0.25) (layer "F.Cu") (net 6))
 (segment (start 165.004511 110.394511) (end 166.37 111.76) (width 0.25) (layer "F.Cu") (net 6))
 (segment (start 166.37 114.3) (end 165.195489 113.125489) (width 0.25) (layer "F.Cu") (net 4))
 (segment (start 62.134511 113.125489) (end 60.96 114.3) (width 0.25) (layer "F.Cu") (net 4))
 (segment (start 165.195489 113.125489) (end 62.134511 113.125489) (width 0.25) (layer "F.Cu") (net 4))
 (segment (start 104.14 53.34) (end 106.68 53.34) (width 0.25) (layer "F.Cu") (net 30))
 (segment (start 106.68 53.34) (end 109.22 55.88) (width 0.25) (layer "F.Cu") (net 30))
 (segment (start 83.82 52.07) (end 88.9 52.07) (width 0.25) (layer "F.Cu") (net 30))
 (segment (start 88.9 52.07) (end 97.79 52.07) (width 0.25) (layer "F.Cu") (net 30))
 (segment (start 97.79 52.07) (end 101.6 55.88) (width 0.25) (layer "F.Cu") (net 30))
 (segment (start 101.6 55.88) (end 104.14 53.34) (width 0.25) (layer "F.Cu") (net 30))
 (segment (start 105.41 59.69) (end 101.6 55.88) (width 0.25) (layer "B.Cu") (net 30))
 (segment (start 105.41 67.83) (end 105.41 59.69) (width 0.25) (layer "B.Cu") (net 30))
 (segment (start 140.97 62.23) (end 132.08 53.34) (width 0.25) (layer "B.Cu") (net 28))
 (segment (start 140.97 67.83) (end 140.97 62.23) (width 0.25) (layer "B.Cu") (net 28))
 (segment (start 132.08 50.8) (end 101.6 50.8) (width 0.25) (layer "F.Cu") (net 29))
 (via (at 101.6 50.8) (size 0.8) (drill 0.4) (layers "F.Cu" "B.Cu") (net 29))
 (segment (start 101.6 50.8) (end 100.475489 51.924511) (width 0.25) (layer "B.Cu") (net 29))
 (segment (start 100.475489 65.435489) (end 102.87 67.83) (width 0.25) (layer "B.Cu") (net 29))
 (segment (start 100.475489 51.924511) (end 100.475489 65.435489) (width 0.25) (layer "B.Cu") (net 29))
 (segment (start 107.95 57.15) (end 106.68 55.88) (width 0.25) (layer "B.Cu") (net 31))
 (segment (start 107.95 67.83) (end 107.95 57.15) (width 0.25) (layer "B.Cu") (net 31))
 (segment (start 110.49 59.69) (end 114.3 55.88) (width 0.25) (layer "B.Cu") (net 32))
 (segment (start 110.49 67.83) (end 110.49 59.69) (width 0.25) (layer "B.Cu") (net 32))
 (segment (start 166.37 71.12) (end 165.1 69.85) (width 0.25) (layer "F.Cu") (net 2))
 (segment (start 78.74 81.28) (end 148.59 81.28) (width 0.25) (layer "F.Cu") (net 2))
 (segment (start 67.31 69.85) (end 78.74 81.28) (width 0.25) (layer "F.Cu") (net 2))
 (segment (start 160.02 69.85) (end 148.59 81.28) (width 0.25) (layer "F.Cu") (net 2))
 (segment (start 60.96 71.12) (end 62.23 69.85) (width 0.25) (layer "F.Cu") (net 2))
 (segment (start 62.23 69.85) (end 67.31 69.85) (width 0.25) (layer "F.Cu") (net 2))
 (segment (start 165.1 69.85) (end 160.02 69.85) (width 0.25) (layer "F.Cu") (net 2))
 (segment (start 60.96 86.36) (end 62.134511 85.185489) (width 0.25) (layer "F.Cu") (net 16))
 (segment (start 165.195489 85.185489) (end 166.37 86.36) (width 0.25) (layer "F.Cu") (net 16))
 (segment (start 62.134511 85.185489) (end 165.195489 85.185489) (width 0.25) (layer "F.Cu") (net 16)))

